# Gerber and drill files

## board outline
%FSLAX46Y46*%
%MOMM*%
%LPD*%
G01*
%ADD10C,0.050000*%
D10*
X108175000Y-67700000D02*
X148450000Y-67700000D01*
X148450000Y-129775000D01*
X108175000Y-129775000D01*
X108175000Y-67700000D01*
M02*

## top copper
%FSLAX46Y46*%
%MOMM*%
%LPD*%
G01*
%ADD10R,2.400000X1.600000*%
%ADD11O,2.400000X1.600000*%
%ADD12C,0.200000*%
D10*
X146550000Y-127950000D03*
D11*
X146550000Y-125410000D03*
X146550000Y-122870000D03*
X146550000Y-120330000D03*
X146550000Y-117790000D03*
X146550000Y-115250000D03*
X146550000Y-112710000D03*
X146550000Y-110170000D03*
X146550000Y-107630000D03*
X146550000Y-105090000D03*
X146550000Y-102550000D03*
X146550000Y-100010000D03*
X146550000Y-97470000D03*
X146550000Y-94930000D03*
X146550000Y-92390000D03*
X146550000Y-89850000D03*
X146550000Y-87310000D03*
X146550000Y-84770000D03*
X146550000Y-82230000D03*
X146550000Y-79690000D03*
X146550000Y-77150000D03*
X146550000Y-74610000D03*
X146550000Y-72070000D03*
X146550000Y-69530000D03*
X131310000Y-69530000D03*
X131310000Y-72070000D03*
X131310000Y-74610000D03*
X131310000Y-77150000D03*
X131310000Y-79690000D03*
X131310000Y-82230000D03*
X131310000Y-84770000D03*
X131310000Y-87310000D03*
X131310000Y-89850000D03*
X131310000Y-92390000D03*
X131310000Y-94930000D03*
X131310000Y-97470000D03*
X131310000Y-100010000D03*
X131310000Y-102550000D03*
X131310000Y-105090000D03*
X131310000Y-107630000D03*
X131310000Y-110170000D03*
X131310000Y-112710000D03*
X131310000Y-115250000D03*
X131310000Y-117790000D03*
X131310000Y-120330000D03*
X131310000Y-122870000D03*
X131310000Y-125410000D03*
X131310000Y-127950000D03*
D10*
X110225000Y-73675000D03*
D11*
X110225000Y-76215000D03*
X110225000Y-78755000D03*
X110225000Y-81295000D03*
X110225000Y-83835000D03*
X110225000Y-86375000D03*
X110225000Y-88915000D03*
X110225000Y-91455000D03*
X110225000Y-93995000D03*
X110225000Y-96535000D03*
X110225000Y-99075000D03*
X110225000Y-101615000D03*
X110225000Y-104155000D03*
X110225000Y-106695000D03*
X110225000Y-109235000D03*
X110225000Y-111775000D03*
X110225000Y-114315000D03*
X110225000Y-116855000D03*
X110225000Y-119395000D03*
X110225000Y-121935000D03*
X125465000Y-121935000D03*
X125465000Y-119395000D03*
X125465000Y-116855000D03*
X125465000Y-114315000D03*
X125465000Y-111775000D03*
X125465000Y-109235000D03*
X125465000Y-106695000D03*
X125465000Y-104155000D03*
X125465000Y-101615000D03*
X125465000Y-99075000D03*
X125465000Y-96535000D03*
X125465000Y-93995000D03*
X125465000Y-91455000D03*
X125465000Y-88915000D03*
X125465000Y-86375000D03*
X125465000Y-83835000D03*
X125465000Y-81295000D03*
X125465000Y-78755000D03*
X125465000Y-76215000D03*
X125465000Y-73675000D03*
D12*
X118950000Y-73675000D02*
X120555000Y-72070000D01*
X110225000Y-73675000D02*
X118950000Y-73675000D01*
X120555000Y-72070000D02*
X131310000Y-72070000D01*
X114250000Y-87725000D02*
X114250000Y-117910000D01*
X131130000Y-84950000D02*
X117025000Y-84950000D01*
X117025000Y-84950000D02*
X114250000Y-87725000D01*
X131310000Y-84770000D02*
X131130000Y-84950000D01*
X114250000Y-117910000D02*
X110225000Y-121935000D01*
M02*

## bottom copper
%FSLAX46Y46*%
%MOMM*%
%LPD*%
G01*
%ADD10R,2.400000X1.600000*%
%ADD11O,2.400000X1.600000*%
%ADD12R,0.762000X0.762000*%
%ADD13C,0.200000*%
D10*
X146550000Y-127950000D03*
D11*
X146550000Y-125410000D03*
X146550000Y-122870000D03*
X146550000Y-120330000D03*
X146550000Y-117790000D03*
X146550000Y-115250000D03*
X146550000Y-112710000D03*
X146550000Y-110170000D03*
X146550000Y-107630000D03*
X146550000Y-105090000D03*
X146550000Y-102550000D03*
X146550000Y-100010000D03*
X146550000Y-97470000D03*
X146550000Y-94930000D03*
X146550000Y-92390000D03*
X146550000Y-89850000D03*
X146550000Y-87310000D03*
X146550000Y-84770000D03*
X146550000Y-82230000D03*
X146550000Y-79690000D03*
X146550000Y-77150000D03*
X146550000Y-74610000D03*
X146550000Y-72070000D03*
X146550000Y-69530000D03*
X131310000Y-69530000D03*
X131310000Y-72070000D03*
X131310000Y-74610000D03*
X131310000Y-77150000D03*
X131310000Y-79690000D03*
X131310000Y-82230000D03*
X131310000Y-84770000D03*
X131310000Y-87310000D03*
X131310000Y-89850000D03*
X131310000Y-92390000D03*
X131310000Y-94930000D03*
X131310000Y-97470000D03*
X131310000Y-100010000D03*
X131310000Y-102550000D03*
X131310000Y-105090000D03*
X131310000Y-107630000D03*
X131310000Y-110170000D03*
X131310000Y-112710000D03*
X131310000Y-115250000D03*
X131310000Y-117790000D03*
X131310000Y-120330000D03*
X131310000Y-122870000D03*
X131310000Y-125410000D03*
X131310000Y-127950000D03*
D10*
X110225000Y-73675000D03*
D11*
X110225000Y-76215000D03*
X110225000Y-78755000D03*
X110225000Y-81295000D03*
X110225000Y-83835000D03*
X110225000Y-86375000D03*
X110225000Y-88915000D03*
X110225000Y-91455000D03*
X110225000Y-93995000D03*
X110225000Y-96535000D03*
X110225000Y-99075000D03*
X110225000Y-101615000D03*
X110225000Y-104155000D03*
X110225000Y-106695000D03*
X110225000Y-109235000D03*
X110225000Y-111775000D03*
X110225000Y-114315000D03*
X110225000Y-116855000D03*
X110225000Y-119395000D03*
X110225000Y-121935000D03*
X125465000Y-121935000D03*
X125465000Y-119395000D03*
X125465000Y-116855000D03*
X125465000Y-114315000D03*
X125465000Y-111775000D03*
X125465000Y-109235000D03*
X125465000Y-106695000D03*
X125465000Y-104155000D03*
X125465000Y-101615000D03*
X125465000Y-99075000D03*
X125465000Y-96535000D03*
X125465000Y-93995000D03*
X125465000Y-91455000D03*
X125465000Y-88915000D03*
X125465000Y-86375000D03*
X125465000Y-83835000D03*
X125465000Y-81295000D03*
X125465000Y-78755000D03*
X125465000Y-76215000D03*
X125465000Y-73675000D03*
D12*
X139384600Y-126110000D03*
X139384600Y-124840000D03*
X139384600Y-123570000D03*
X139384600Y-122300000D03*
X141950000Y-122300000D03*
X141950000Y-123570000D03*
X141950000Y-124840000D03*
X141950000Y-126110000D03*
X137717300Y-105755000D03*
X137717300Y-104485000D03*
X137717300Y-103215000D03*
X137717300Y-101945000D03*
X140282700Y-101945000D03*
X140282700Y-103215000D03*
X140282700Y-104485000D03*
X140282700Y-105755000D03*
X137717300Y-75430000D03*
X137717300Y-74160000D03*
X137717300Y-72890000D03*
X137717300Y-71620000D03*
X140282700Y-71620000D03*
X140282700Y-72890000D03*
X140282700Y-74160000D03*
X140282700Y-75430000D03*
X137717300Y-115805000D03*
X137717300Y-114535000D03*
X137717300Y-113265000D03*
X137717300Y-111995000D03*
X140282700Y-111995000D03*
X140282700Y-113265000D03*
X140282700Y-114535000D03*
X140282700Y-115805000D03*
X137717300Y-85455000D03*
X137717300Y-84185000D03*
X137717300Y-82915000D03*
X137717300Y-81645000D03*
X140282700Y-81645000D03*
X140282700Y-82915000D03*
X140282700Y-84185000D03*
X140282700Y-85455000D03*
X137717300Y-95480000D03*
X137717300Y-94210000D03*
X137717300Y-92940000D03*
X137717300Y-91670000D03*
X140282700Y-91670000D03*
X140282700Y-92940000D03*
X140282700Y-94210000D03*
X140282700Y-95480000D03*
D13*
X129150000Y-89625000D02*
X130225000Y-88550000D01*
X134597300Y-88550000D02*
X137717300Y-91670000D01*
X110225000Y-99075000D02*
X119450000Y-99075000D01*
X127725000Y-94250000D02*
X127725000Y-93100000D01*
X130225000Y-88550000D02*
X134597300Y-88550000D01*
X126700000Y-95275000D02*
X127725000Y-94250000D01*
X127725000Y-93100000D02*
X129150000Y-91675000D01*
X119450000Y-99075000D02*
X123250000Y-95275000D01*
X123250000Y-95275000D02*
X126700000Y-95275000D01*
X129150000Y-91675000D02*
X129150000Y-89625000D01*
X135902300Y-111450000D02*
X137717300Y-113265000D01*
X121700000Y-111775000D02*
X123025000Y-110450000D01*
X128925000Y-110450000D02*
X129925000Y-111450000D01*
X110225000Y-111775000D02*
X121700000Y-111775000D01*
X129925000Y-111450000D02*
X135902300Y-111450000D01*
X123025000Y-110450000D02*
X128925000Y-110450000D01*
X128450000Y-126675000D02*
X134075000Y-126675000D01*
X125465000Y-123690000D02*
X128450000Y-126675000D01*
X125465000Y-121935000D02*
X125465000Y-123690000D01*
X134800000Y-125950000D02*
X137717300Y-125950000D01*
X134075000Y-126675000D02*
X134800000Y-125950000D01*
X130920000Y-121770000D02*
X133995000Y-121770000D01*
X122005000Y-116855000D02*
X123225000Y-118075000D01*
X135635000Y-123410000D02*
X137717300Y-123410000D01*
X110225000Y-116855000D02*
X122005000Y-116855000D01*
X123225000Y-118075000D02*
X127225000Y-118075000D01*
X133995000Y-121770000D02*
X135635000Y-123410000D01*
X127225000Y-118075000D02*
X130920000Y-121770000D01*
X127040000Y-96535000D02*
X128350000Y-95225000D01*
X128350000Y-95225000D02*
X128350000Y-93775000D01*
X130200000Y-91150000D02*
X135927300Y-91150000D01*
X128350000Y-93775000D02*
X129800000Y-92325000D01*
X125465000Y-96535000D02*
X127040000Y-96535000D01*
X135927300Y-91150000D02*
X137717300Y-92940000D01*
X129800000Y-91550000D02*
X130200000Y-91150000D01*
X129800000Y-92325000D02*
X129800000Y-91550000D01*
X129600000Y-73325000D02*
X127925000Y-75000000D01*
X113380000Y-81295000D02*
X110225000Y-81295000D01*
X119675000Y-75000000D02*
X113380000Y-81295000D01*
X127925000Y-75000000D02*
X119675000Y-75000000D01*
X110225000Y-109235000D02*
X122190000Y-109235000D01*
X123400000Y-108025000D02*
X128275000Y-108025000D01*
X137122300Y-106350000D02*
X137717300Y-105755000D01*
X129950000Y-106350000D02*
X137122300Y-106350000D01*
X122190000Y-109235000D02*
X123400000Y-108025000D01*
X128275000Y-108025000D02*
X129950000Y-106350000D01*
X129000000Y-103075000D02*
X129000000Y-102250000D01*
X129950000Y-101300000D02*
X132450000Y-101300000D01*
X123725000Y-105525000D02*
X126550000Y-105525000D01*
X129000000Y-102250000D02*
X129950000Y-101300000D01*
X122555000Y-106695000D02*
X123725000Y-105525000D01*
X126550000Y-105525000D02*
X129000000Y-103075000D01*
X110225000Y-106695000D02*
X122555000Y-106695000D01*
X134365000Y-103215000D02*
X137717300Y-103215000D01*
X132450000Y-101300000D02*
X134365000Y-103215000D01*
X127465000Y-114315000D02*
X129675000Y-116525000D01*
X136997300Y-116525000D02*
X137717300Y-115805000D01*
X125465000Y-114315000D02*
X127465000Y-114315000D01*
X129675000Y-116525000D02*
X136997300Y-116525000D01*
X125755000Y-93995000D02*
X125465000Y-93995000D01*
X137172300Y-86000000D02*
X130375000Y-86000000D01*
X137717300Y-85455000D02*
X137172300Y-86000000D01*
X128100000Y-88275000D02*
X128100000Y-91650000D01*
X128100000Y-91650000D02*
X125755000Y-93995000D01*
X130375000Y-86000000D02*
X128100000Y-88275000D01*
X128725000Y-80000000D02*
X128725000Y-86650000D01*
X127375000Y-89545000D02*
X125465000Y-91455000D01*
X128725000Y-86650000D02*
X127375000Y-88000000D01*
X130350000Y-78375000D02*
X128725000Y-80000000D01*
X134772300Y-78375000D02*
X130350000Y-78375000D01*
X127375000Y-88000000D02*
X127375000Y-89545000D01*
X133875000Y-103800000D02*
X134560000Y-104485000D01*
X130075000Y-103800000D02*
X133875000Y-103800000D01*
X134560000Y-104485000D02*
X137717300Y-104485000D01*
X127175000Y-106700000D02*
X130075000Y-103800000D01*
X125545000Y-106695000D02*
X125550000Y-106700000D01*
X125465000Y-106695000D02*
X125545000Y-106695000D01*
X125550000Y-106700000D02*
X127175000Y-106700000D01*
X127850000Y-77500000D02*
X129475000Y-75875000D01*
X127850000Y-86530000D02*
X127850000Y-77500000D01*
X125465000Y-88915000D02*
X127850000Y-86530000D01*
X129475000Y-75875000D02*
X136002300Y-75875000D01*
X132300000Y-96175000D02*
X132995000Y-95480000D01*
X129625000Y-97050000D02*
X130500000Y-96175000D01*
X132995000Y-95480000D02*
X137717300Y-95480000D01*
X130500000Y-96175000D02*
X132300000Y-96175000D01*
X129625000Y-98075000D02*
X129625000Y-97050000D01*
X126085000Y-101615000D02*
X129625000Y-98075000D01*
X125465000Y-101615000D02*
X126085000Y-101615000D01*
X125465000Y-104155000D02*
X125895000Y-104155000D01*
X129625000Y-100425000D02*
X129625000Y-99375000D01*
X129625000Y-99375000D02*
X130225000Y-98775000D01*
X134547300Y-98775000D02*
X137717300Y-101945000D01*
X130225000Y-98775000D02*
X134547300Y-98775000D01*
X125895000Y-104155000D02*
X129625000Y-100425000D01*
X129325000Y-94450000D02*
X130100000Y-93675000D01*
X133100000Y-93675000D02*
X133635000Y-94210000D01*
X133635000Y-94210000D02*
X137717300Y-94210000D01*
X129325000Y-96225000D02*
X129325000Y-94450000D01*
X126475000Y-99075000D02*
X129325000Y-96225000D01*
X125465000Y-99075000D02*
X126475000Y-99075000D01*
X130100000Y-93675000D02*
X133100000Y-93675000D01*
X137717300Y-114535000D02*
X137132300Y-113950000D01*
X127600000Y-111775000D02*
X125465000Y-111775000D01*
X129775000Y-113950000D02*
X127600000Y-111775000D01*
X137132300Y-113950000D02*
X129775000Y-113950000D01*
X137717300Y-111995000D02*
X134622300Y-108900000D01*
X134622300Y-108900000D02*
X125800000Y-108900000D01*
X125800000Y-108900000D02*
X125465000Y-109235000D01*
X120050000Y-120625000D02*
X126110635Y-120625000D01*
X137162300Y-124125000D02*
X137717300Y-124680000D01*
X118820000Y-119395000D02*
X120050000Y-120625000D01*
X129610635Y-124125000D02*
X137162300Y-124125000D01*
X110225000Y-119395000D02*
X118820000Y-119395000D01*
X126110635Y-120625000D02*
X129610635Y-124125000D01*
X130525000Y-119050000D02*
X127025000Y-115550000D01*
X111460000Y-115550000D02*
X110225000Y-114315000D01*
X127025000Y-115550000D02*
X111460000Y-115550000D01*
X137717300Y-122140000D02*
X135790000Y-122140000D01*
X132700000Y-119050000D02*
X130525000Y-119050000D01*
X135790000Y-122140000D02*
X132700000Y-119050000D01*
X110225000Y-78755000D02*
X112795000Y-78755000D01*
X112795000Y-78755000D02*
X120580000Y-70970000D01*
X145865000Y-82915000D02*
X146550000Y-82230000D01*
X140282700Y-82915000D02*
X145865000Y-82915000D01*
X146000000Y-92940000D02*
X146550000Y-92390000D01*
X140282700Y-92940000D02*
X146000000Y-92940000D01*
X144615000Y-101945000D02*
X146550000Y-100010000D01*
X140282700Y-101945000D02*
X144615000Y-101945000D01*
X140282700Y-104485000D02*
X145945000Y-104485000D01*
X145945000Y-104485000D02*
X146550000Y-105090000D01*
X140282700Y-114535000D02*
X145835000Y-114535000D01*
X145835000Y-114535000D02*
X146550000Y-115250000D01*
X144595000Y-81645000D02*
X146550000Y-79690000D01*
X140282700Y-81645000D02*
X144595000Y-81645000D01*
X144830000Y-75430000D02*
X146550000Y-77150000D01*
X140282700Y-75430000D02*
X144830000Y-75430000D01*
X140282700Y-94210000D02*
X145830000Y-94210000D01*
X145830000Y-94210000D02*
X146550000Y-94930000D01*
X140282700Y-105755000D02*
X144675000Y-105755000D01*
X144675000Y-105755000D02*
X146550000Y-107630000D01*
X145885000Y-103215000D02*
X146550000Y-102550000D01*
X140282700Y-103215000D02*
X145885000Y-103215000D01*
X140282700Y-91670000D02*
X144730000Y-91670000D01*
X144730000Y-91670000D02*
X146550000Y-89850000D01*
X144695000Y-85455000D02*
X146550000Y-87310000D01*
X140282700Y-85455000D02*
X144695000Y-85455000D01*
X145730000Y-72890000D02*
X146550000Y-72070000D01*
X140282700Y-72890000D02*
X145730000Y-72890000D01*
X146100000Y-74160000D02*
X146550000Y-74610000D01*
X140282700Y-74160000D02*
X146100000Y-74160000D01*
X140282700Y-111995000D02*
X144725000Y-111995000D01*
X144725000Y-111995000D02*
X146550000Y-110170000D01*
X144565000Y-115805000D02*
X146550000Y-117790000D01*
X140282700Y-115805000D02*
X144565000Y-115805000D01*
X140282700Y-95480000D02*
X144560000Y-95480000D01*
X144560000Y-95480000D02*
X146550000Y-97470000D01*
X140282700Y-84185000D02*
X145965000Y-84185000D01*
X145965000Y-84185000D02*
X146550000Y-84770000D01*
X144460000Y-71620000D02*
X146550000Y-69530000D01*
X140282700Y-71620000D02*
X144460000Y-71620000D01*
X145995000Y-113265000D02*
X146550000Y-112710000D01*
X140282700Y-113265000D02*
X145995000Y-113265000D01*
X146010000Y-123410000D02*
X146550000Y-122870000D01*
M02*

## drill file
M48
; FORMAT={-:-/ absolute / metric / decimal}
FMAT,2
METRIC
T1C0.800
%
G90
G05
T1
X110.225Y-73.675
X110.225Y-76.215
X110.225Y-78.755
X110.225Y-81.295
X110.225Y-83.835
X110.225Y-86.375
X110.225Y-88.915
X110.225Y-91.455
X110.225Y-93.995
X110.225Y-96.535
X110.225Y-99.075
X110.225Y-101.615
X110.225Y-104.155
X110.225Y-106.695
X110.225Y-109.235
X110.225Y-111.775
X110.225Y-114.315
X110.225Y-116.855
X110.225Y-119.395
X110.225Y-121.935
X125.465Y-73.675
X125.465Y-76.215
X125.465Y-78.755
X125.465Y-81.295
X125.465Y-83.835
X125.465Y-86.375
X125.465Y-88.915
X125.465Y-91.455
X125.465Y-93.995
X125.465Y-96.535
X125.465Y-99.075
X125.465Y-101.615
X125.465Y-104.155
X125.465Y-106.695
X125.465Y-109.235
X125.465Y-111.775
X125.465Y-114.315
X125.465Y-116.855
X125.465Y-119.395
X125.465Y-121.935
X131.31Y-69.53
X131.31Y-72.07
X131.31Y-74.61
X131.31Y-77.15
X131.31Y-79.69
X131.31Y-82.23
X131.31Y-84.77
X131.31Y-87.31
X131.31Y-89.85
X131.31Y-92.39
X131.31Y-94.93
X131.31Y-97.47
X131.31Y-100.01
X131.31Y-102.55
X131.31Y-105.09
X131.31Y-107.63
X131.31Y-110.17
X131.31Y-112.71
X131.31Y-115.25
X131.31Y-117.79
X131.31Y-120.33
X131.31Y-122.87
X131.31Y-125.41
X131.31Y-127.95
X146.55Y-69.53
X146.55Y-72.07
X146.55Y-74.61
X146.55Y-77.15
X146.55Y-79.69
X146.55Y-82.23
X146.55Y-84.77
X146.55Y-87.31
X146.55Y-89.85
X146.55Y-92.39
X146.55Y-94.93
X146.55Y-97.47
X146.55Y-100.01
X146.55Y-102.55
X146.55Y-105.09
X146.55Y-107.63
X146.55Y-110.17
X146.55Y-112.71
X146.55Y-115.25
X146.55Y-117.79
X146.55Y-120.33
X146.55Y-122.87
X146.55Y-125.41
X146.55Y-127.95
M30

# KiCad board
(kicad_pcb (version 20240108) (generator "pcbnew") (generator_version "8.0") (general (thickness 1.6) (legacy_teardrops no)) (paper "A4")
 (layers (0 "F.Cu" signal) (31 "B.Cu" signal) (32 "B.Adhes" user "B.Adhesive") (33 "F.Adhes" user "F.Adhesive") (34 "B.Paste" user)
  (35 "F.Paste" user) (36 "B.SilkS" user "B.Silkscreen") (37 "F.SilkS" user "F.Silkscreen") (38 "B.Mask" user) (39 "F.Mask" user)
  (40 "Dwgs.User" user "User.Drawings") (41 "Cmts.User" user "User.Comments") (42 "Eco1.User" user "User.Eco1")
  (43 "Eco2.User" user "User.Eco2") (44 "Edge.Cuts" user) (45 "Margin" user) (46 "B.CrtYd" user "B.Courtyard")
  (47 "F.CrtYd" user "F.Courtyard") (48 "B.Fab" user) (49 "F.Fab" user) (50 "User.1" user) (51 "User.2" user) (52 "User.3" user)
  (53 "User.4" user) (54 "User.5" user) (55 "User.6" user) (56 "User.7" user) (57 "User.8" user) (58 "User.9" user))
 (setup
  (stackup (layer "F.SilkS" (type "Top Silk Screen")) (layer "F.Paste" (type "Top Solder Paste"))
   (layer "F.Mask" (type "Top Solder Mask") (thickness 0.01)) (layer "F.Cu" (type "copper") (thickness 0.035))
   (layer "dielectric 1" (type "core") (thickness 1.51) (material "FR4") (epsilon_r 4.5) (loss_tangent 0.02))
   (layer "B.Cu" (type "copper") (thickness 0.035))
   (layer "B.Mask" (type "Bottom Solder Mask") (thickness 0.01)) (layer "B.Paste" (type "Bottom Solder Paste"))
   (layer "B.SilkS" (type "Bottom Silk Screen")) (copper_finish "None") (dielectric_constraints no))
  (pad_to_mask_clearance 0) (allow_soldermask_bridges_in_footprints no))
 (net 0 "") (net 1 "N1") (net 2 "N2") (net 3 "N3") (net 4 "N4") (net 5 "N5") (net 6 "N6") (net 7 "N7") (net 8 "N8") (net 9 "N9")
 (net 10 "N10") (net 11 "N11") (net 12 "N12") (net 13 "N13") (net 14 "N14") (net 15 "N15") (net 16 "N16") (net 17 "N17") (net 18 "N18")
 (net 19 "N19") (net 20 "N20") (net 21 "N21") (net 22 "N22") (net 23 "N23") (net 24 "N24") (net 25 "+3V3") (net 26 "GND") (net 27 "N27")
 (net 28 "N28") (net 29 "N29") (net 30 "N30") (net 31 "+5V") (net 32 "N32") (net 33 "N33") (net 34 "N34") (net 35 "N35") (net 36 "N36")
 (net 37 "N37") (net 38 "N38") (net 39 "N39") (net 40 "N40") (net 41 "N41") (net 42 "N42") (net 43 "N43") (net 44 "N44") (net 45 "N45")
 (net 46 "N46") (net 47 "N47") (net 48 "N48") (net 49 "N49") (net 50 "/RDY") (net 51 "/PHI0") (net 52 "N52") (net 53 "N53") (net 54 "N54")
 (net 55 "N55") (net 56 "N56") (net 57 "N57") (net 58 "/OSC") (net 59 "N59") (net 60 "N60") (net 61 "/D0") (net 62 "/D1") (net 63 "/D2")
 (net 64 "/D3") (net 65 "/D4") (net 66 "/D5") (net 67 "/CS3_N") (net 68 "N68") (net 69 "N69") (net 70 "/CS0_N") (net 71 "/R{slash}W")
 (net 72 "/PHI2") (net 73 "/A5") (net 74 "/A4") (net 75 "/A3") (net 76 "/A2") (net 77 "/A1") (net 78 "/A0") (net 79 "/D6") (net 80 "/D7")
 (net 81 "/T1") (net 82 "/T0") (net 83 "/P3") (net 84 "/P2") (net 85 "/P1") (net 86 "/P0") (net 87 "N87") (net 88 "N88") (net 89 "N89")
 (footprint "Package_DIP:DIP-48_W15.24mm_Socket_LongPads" (layer "F.Cu") (at 146.55 127.95 180)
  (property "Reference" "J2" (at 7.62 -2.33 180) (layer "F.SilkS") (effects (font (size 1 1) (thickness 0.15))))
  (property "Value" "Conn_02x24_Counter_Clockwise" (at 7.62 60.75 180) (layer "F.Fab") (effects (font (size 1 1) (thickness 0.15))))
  (pad "1" thru_hole rect (at 0 0 180) (size 2.4 1.6) (drill 0.8) (layers "*.Cu" "*.Mask") (remove_unused_layers no) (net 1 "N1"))
  (pad "2" thru_hole oval (at 0 2.54 180) (size 2.4 1.6) (drill 0.8) (layers "*.Cu" "*.Mask") (remove_unused_layers no) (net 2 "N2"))
  (pad "3" thru_hole oval (at 0 5.08 180) (size 2.4 1.6) (drill 0.8) (layers "*.Cu" "*.Mask") (remove_unused_layers no) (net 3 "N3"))
  (pad "4" thru_hole oval (at 0 7.62 180) (size 2.4 1.6) (drill 0.8) (layers "*.Cu" "*.Mask") (remove_unused_layers no) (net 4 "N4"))
  (pad "5" thru_hole oval (at 0 10.16 180) (size 2.4 1.6) (drill 0.8) (layers "*.Cu" "*.Mask") (remove_unused_layers no) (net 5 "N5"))
  (pad "6" thru_hole oval (at 0 12.7 180) (size 2.4 1.6) (drill 0.8) (layers "*.Cu" "*.Mask") (remove_unused_layers no) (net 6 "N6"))
  (pad "7" thru_hole oval (at 0 15.24 180) (size 2.4 1.6) (drill 0.8) (layers "*.Cu" "*.Mask") (remove_unused_layers no) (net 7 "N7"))
  (pad "8" thru_hole oval (at 0 17.78 180) (size 2.4 1.6) (drill 0.8) (layers "*.Cu" "*.Mask") (remove_unused_layers no) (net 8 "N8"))
  (pad "9" thru_hole oval (at 0 20.32 180) (size 2.4 1.6) (drill 0.8) (layers "*.Cu" "*.Mask") (remove_unused_layers no) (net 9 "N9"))
  (pad "10" thru_hole oval (at 0 22.86 180) (size 2.4 1.6) (drill 0.8) (layers "*.Cu" "*.Mask") (remove_unused_layers no) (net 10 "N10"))
  (pad "11" thru_hole oval (at 0 25.4 180) (size 2.4 1.6) (drill 0.8) (layers "*.Cu" "*.Mask") (remove_unused_layers no) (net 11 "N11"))
  (pad "12" thru_hole oval (at 0 27.94 180) (size 2.4 1.6) (drill 0.8) (layers "*.Cu" "*.Mask") (remove_unused_layers no) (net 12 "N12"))
  (pad "13" thru_hole oval (at 0 30.48 180) (size 2.4 1.6) (drill 0.8) (layers "*.Cu" "*.Mask") (remove_unused_layers no) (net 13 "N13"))
  (pad "14" thru_hole oval (at 0 33.02 180) (size 2.4 1.6) (drill 0.8) (layers "*.Cu" "*.Mask") (remove_unused_layers no) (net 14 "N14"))
  (pad "15" thru_hole oval (at 0 35.56 180) (size 2.4 1.6) (drill 0.8) (layers "*.Cu" "*.Mask") (remove_unused_layers no) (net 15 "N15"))
  (pad "16" thru_hole oval (at 0 38.1 180) (size 2.4 1.6) (drill 0.8) (layers "*.Cu" "*.Mask") (remove_unused_layers no) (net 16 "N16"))
  (pad "17" thru_hole oval (at 0 40.64 180) (size 2.4 1.6) (drill 0.8) (layers "*.Cu" "*.Mask") (remove_unused_layers no) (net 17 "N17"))
  (pad "18" thru_hole oval (at 0 43.18 180) (size 2.4 1.6) (drill 0.8) (layers "*.Cu" "*.Mask") (remove_unused_layers no) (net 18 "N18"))
  (pad "19" thru_hole oval (at 0 45.72 180) (size 2.4 1.6) (drill 0.8) (layers "*.Cu" "*.Mask") (remove_unused_layers no) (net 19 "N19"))
  (pad "20" thru_hole oval (at 0 48.26 180) (size 2.4 1.6) (drill 0.8) (layers "*.Cu" "*.Mask") (remove_unused_layers no) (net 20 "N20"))
  (pad "21" thru_hole oval (at 0 50.8 180) (size 2.4 1.6) (drill 0.8) (layers "*.Cu" "*.Mask") (remove_unused_layers no) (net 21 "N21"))
  (pad "22" thru_hole oval (at 0 53.34 180) (size 2.4 1.6) (drill 0.8) (layers "*.Cu" "*.Mask") (remove_unused_layers no) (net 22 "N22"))
  (pad "23" thru_hole oval (at 0 55.88 180) (size 2.4 1.6) (drill 0.8) (layers "*.Cu" "*.Mask") (remove_unused_layers no) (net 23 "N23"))
  (pad "24" thru_hole oval (at 0 58.42 180) (size 2.4 1.6) (drill 0.8) (layers "*.Cu" "*.Mask") (remove_unused_layers no) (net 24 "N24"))
  (pad "25" thru_hole oval (at 15.24 58.42 180) (size 2.4 1.6) (drill 0.8) (layers "*.Cu" "*.Mask") (remove_unused_layers no)
   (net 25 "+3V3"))
  (pad "26" thru_hole oval (at 15.24 55.88 180) (size 2.4 1.6) (drill 0.8) (layers "*.Cu" "*.Mask") (remove_unused_layers no) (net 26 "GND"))
  (pad "27" thru_hole oval (at 15.24 53.34 180) (size 2.4 1.6) (drill 0.8) (layers "*.Cu" "*.Mask") (remove_unused_layers no) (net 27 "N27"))
  (pad "28" thru_hole oval (at 15.24 50.8 180) (size 2.4 1.6) (drill 0.8) (layers "*.Cu" "*.Mask") (remove_unused_layers no) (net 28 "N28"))
  (pad "29" thru_hole oval (at 15.24 48.26 180) (size 2.4 1.6) (drill 0.8) (layers "*.Cu" "*.Mask") (remove_unused_layers no) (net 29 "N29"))
  (pad "30" thru_hole oval (at 15.24 45.72 180) (size 2.4 1.6) (drill 0.8) (layers "*.Cu" "*.Mask") (remove_unused_layers no) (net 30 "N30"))
  (pad "31" thru_hole oval (at 15.24 43.18 180) (size 2.4 1.6) (drill 0.8) (layers "*.Cu" "*.Mask") (remove_unused_layers no) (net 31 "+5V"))
  (pad "32" thru_hole oval (at 15.24 40.64 180) (size 2.4 1.6) (drill 0.8) (layers "*.Cu" "*.Mask") (remove_unused_layers no) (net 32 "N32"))
  (pad "33" thru_hole oval (at 15.24 38.1 180) (size 2.4 1.6) (drill 0.8) (layers "*.Cu" "*.Mask") (remove_unused_layers no) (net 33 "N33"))
  (pad "34" thru_hole oval (at 15.24 35.56 180) (size 2.4 1.6) (drill 0.8) (layers "*.Cu" "*.Mask") (remove_unused_layers no) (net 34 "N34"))
  (pad "35" thru_hole oval (at 15.24 33.02 180) (size 2.4 1.6) (drill 0.8) (layers "*.Cu" "*.Mask") (remove_unused_layers no) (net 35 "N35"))
  (pad "36" thru_hole oval (at 15.24 30.48 180) (size 2.4 1.6) (drill 0.8) (layers "*.Cu" "*.Mask") (remove_unused_layers no) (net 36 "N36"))
  (pad "37" thru_hole oval (at 15.24 27.94 180) (size 2.4 1.6) (drill 0.8) (layers "*.Cu" "*.Mask") (remove_unused_layers no) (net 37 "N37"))
  (pad "38" thru_hole oval (at 15.24 25.4 180) (size 2.4 1.6) (drill 0.8) (layers "*.Cu" "*.Mask") (remove_unused_layers no) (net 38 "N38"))
  (pad "39" thru_hole oval (at 15.24 22.86 180) (size 2.4 1.6) (drill 0.8) (layers "*.Cu" "*.Mask") (remove_unused_layers no) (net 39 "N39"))
  (pad "40" thru_hole oval (at 15.24 20.32 180) (size 2.4 1.6) (drill 0.8) (layers "*.Cu" "*.Mask") (remove_unused_layers no) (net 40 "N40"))
  (pad "41" thru_hole oval (at 15.24 17.78 180) (size 2.4 1.6) (drill 0.8) (layers "*.Cu" "*.Mask") (remove_unused_layers no) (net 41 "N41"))
  (pad "42" thru_hole oval (at 15.24 15.24 180) (size 2.4 1.6) (drill 0.8) (layers "*.Cu" "*.Mask") (remove_unused_layers no) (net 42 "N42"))
  (pad "43" thru_hole oval (at 15.24 12.7 180) (size 2.4 1.6) (drill 0.8) (layers "*.Cu" "*.Mask") (remove_unused_layers no) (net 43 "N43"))
  (pad "44" thru_hole oval (at 15.24 10.16 180) (size 2.4 1.6) (drill 0.8) (layers "*.Cu" "*.Mask") (remove_unused_layers no) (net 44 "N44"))
  (pad "45" thru_hole oval (at 15.24 7.62 180) (size 2.4 1.6) (drill 0.8) (layers "*.Cu" "*.Mask") (remove_unused_layers no) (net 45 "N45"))
  (pad "46" thru_hole oval (at 15.24 5.08 180) (size 2.4 1.6) (drill 0.8) (layers "*.Cu" "*.Mask") (remove_unused_layers no) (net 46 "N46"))
  (pad "47" thru_hole oval (at 15.24 2.54 180) (size 2.4 1.6) (drill 0.8) (layers "*.Cu" "*.Mask") (remove_unused_layers no) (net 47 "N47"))
  (pad "48" thru_hole oval (at 15.24 0 180) (size 2.4 1.6) (drill 0.8) (layers "*.Cu" "*.Mask") (remove_unused_layers no) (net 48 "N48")))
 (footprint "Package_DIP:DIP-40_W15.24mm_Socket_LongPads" (layer "F.Cu") (at 110.225 73.675)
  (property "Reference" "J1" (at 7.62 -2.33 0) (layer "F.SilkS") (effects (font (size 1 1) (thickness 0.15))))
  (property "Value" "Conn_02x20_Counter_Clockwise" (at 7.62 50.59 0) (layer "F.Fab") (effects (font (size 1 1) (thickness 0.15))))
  (pad "1" thru_hole rect (at 0 0) (size 2.4 1.6) (drill 0.8) (layers "*.Cu" "*.Mask") (remove_unused_layers no) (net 26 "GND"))
  (pad "2" thru_hole oval (at 0 2.54) (size 2.4 1.6) (drill 0.8) (layers "*.Cu" "*.Mask") (remove_unused_layers no) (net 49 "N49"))
  (pad "3" thru_hole oval (at 0 5.08) (size 2.4 1.6) (drill 0.8) (layers "*.Cu" "*.Mask") (remove_unused_layers no) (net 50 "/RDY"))
  (pad "4" thru_hole oval (at 0 7.62) (size 2.4 1.6) (drill 0.8) (layers "*.Cu" "*.Mask") (remove_unused_layers no) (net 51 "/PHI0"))
  (pad "5" thru_hole oval (at 0 10.16) (size 2.4 1.6) (drill 0.8) (layers "*.Cu" "*.Mask") (remove_unused_layers no) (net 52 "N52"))
  (pad "6" thru_hole oval (at 0 12.7) (size 2.4 1.6) (drill 0.8) (layers "*.Cu" "*.Mask") (remove_unused_layers no) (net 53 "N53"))
  (pad "7" thru_hole oval (at 0 15.24) (size 2.4 1.6) (drill 0.8) (layers "*.Cu" "*.Mask") (remove_unused_layers no) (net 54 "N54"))
  (pad "8" thru_hole oval (at 0 17.78) (size 2.4 1.6) (drill 0.8) (layers "*.Cu" "*.Mask") (remove_unused_layers no) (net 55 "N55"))
  (pad "9" thru_hole oval (at 0 20.32) (size 2.4 1.6) (drill 0.8) (layers "*.Cu" "*.Mask") (remove_unused_layers no) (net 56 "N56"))
  (pad "10" thru_hole oval (at 0 22.86) (size 2.4 1.6) (drill 0.8) (layers "*.Cu" "*.Mask") (remove_unused_layers no) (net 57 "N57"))
  (pad "11" thru_hole oval (at 0 25.4) (size 2.4 1.6) (drill 0.8) (layers "*.Cu" "*.Mask") (remove_unused_layers no) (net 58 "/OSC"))
  (pad "12" thru_hole oval (at 0 27.94) (size 2.4 1.6) (drill 0.8) (layers "*.Cu" "*.Mask") (remove_unused_layers no) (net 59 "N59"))
  (pad "13" thru_hole oval (at 0 30.48) (size 2.4 1.6) (drill 0.8) (layers "*.Cu" "*.Mask") (remove_unused_layers no) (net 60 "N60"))
  (pad "14" thru_hole oval (at 0 33.02) (size 2.4 1.6) (drill 0.8) (layers "*.Cu" "*.Mask") (remove_unused_layers no) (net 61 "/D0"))
  (pad "15" thru_hole oval (at 0 35.56) (size 2.4 1.6) (drill 0.8) (layers "*.Cu" "*.Mask") (remove_unused_layers no) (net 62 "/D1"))
  (pad "16" thru_hole oval (at 0 38.1) (size 2.4 1.6) (drill 0.8) (layers "*.Cu" "*.Mask") (remove_unused_layers no) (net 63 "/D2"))
  (pad "17" thru_hole oval (at 0 40.64) (size 2.4 1.6) (drill 0.8) (layers "*.Cu" "*.Mask") (remove_unused_layers no) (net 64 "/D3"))
  (pad "18" thru_hole oval (at 0 43.18) (size 2.4 1.6) (drill 0.8) (layers "*.Cu" "*.Mask") (remove_unused_layers no) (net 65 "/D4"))
  (pad "19" thru_hole oval (at 0 45.72) (size 2.4 1.6) (drill 0.8) (layers "*.Cu" "*.Mask") (remove_unused_layers no) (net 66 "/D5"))
  (pad "20" thru_hole oval (at 0 48.26) (size 2.4 1.6) (drill 0.8) (layers "*.Cu" "*.Mask") (remove_unused_layers no) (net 31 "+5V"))
  (pad "21" thru_hole oval (at 15.24 48.26) (size 2.4 1.6) (drill 0.8) (layers "*.Cu" "*.Mask") (remove_unused_layers no) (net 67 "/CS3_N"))
  (pad "22" thru_hole oval (at 15.24 45.72) (size 2.4 1.6) (drill 0.8) (layers "*.Cu" "*.Mask") (remove_unused_layers no) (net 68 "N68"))
  (pad "23" thru_hole oval (at 15.24 43.18) (size 2.4 1.6) (drill 0.8) (layers "*.Cu" "*.Mask") (remove_unused_layers no) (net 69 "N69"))
  (pad "24" thru_hole oval (at 15.24 40.64) (size 2.4 1.6) (drill 0.8) (layers "*.Cu" "*.Mask") (remove_unused_layers no) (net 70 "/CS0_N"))
  (pad "25" thru_hole oval (at 15.24 38.1) (size 2.4 1.6) (drill 0.8) (layers "*.Cu" "*.Mask") (remove_unused_layers no)
   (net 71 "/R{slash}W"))
  (pad "26" thru_hole oval (at 15.24 35.56) (size 2.4 1.6) (drill 0.8) (layers "*.Cu" "*.Mask") (remove_unused_layers no) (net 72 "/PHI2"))
  (pad "27" thru_hole oval (at 15.24 33.02) (size 2.4 1.6) (drill 0.8) (layers "*.Cu" "*.Mask") (remove_unused_layers no) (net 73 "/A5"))
  (pad "28" thru_hole oval (at 15.24 30.48) (size 2.4 1.6) (drill 0.8) (layers "*.Cu" "*.Mask") (remove_unused_layers no) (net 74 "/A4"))
  (pad "29" thru_hole oval (at 15.24 27.94) (size 2.4 1.6) (drill 0.8) (layers "*.Cu" "*.Mask") (remove_unused_layers no) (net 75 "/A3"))
  (pad "30" thru_hole oval (at 15.24 25.4) (size 2.4 1.6) (drill 0.8) (layers "*.Cu" "*.Mask") (remove_unused_layers no) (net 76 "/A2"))
  (pad "31" thru_hole oval (at 15.24 22.86) (size 2.4 1.6) (drill 0.8) (layers "*.Cu" "*.Mask") (remove_unused_layers no) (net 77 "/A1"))
  (pad "32" thru_hole oval (at 15.24 20.32) (size 2.4 1.6) (drill 0.8) (layers "*.Cu" "*.Mask") (remove_unused_layers no) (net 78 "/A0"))
  (pad "33" thru_hole oval (at 15.24 17.78) (size 2.4 1.6) (drill 0.8) (layers "*.Cu" "*.Mask") (remove_unused_layers no) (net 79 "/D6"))
  (pad "34" thru_hole oval (at 15.24 15.24) (size 2.4 1.6) (drill 0.8) (layers "*.Cu" "*.Mask") (remove_unused_layers no) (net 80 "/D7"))
  (pad "35" thru_hole oval (at 15.24 12.7) (size 2.4 1.6) (drill 0.8) (layers "*.Cu" "*.Mask") (remove_unused_layers no) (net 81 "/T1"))
  (pad "36" thru_hole oval (at 15.24 10.16) (size 2.4 1.6) (drill 0.8) (layers "*.Cu" "*.Mask") (remove_unused_layers no) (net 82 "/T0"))
  (pad "37" thru_hole oval (at 15.24 7.62) (size 2.4 1.6) (drill 0.8) (layers "*.Cu" "*.Mask") (remove_unused_layers no) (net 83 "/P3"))
  (pad "38" thru_hole oval (at 15.24 5.08) (size 2.4 1.6) (drill 0.8) (layers "*.Cu" "*.Mask") (remove_unused_layers no) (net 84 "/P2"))
  (pad "39" thru_hole oval (at 15.24 2.54) (size 2.4 1.6) (drill 0.8) (layers "*.Cu" "*.Mask") (remove_unused_layers no) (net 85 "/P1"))
  (pad "40" thru_hole oval (at 15.24 0) (size 2.4 1.6) (drill 0.8) (layers "*.Cu" "*.Mask") (remove_unused_layers no) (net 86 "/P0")))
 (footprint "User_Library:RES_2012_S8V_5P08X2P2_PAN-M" (layer "B.Cu") (at 140.6673 124.205)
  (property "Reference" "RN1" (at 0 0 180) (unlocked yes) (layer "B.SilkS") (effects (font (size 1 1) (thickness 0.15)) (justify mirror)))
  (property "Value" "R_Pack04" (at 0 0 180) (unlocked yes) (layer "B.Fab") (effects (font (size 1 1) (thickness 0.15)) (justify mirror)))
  (pad "1" smd rect (at -1.2827 1.905) (size 0.762 0.762) (layers "B.Cu" "B.Paste" "B.Mask") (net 30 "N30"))
  (pad "2" smd rect (at -1.2827 0.635) (size 0.762 0.762) (layers "B.Cu" "B.Paste" "B.Mask") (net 29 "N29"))
  (pad "3" smd rect (at -1.2827 -0.635) (size 0.762 0.762) (layers "B.Cu" "B.Paste" "B.Mask") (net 28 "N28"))
  (pad "4" smd rect (at -1.2827 -1.905) (size 0.762 0.762) (layers "B.Cu" "B.Paste" "B.Mask") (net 27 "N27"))
  (pad "5" smd rect (at 1.2827 -1.905) (size 0.762 0.762) (layers "B.Cu" "B.Paste" "B.Mask") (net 64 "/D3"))
  (pad "6" smd rect (at 1.2827 -0.635) (size 0.762 0.762) (layers "B.Cu" "B.Paste" "B.Mask") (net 65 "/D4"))
  (pad "7" smd rect (at 1.2827 0.635) (size 0.762 0.762) (layers "B.Cu" "B.Paste" "B.Mask") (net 66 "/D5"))
  (pad "8" smd rect (at 1.2827 1.905) (size 0.762 0.762) (layers "B.Cu" "B.Paste" "B.Mask") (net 67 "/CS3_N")))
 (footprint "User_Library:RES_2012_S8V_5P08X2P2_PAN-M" (layer "B.Cu") (at 139 103.85)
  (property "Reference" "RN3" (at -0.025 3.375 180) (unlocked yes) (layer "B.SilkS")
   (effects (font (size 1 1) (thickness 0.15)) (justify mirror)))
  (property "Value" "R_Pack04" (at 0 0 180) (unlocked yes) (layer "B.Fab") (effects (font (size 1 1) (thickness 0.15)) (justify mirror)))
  (pad "1" smd rect (at -1.2827 1.905) (size 0.762 0.762) (layers "B.Cu" "B.Paste" "B.Mask") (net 62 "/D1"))
  (pad "2" smd rect (at -1.2827 0.635) (size 0.762 0.762) (layers "B.Cu" "B.Paste" "B.Mask") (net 73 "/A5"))
  (pad "3" smd rect (at -1.2827 -0.635) (size 0.762 0.762) (layers "B.Cu" "B.Paste" "B.Mask") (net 61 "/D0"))
  (pad "4" smd rect (at -1.2827 -1.905) (size 0.762 0.762) (layers "B.Cu" "B.Paste" "B.Mask") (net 74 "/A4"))
  (pad "5" smd rect (at 1.2827 -1.905) (size 0.762 0.762) (layers "B.Cu" "B.Paste" "B.Mask") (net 12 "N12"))
  (pad "6" smd rect (at 1.2827 -0.635) (size 0.762 0.762) (layers "B.Cu" "B.Paste" "B.Mask") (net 11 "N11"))
  (pad "7" smd rect (at 1.2827 0.635) (size 0.762 0.762) (layers "B.Cu" "B.Paste" "B.Mask") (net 10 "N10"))
  (pad "8" smd rect (at 1.2827 1.905) (size 0.762 0.762) (layers "B.Cu" "B.Paste" "B.Mask") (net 9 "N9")))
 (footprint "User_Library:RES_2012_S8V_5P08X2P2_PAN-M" (layer "B.Cu") (at 139 73.525)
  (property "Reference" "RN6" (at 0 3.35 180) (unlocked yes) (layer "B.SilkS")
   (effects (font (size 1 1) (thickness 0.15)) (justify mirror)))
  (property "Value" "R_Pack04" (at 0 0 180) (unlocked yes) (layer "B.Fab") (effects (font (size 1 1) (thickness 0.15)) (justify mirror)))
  (pad "1" smd rect (at -1.2827 1.905) (size 0.762 0.762) (layers "B.Cu" "B.Paste" "B.Mask") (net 50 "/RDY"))
  (pad "2" smd rect (at -1.2827 0.635) (size 0.762 0.762) (layers "B.Cu" "B.Paste" "B.Mask") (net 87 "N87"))
  (pad "3" smd rect (at -1.2827 -0.635) (size 0.762 0.762) (layers "B.Cu" "B.Paste" "B.Mask") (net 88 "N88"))
  (pad "4" smd rect (at -1.2827 -1.905) (size 0.762 0.762) (layers "B.Cu" "B.Paste" "B.Mask") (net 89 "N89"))
  (pad "5" smd rect (at 1.2827 -1.905) (size 0.762 0.762) (layers "B.Cu" "B.Paste" "B.Mask") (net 24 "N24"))
  (pad "6" smd rect (at 1.2827 -0.635) (size 0.762 0.762) (layers "B.Cu" "B.Paste" "B.Mask") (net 23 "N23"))
  (pad "7" smd rect (at 1.2827 0.635) (size 0.762 0.762) (layers "B.Cu" "B.Paste" "B.Mask") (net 22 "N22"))
  (pad "8" smd rect (at 1.2827 1.905) (size 0.762 0.762) (layers "B.Cu" "B.Paste" "B.Mask") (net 21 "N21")))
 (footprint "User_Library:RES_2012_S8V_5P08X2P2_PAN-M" (layer "B.Cu") (at 139 113.9)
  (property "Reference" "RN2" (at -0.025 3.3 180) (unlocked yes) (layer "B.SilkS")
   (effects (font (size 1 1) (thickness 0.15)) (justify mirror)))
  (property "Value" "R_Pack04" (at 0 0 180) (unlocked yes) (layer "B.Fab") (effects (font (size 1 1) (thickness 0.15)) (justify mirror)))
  (pad "1" smd rect (at -1.2827 1.905) (size 0.762 0.762) (layers "B.Cu" "B.Paste" "B.Mask") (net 70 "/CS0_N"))
  (pad "2" smd rect (at -1.2827 0.635) (size 0.762 0.762) (layers "B.Cu" "B.Paste" "B.Mask") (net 71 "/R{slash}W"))
  (pad "3" smd rect (at -1.2827 -0.635) (size 0.762 0.762) (layers "B.Cu" "B.Paste" "B.Mask") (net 63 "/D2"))
  (pad "4" smd rect (at -1.2827 -1.905) (size 0.762 0.762) (layers "B.Cu" "B.Paste" "B.Mask") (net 72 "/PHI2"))
  (pad "5" smd rect (at 1.2827 -1.905) (size 0.762 0.762) (layers "B.Cu" "B.Paste" "B.Mask") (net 8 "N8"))
  (pad "6" smd rect (at 1.2827 -0.635) (size 0.762 0.762) (layers "B.Cu" "B.Paste" "B.Mask") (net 7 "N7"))
  (pad "7" smd rect (at 1.2827 0.635) (size 0.762 0.762) (layers "B.Cu" "B.Paste" "B.Mask") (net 6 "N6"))
  (pad "8" smd rect (at 1.2827 1.905) (size 0.762 0.762) (layers "B.Cu" "B.Paste" "B.Mask") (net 5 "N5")))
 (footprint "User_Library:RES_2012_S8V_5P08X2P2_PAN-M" (layer "B.Cu") (at 139 83.55)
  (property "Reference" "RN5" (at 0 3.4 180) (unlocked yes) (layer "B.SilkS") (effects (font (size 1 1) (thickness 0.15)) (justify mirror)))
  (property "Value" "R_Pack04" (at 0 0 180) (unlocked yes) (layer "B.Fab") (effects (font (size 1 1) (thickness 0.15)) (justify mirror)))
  (pad "1" smd rect (at -1.2827 1.905) (size 0.762 0.762) (layers "B.Cu" "B.Paste" "B.Mask") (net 78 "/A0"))
  (pad "2" smd rect (at -1.2827 0.635) (size 0.762 0.762) (layers "B.Cu" "B.Paste" "B.Mask") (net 79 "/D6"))
  (pad "3" smd rect (at -1.2827 -0.635) (size 0.762 0.762) (layers "B.Cu" "B.Paste" "B.Mask") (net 80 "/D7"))
  (pad "4" smd rect (at -1.2827 -1.905) (size 0.762 0.762) (layers "B.Cu" "B.Paste" "B.Mask") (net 51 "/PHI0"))
  (pad "5" smd rect (at 1.2827 -1.905) (size 0.762 0.762) (layers "B.Cu" "B.Paste" "B.Mask") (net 20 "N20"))
  (pad "6" smd rect (at 1.2827 -0.635) (size 0.762 0.762) (layers "B.Cu" "B.Paste" "B.Mask") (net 19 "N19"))
  (pad "7" smd rect (at 1.2827 0.635) (size 0.762 0.762) (layers "B.Cu" "B.Paste" "B.Mask") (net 18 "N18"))
  (pad "8" smd rect (at 1.2827 1.905) (size 0.762 0.762) (layers "B.Cu" "B.Paste" "B.Mask") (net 17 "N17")))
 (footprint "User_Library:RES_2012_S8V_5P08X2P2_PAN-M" (layer "B.Cu") (at 139 93.575)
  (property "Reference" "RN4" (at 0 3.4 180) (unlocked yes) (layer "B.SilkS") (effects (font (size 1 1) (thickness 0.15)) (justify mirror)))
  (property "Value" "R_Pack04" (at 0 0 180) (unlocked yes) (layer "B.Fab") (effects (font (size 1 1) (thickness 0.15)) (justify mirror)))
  (pad "1" smd rect (at -1.2827 1.905) (size 0.762 0.762) (layers "B.Cu" "B.Paste" "B.Mask") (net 75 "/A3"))
  (pad "2" smd rect (at -1.2827 0.635) (size 0.762 0.762) (layers "B.Cu" "B.Paste" "B.Mask") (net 76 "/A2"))
  (pad "3" smd rect (at -1.2827 -0.635) (size 0.762 0.762) (layers "B.Cu" "B.Paste" "B.Mask") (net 77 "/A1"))
  (pad "4" smd rect (at -1.2827 -1.905) (size 0.762 0.762) (layers "B.Cu" "B.Paste" "B.Mask") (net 58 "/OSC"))
  (pad "5" smd rect (at 1.2827 -1.905) (size 0.762 0.762) (layers "B.Cu" "B.Paste" "B.Mask") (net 16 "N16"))
  (pad "6" smd rect (at 1.2827 -0.635) (size 0.762 0.762) (layers "B.Cu" "B.Paste" "B.Mask") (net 15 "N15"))
  (pad "7" smd rect (at 1.2827 0.635) (size 0.762 0.762) (layers "B.Cu" "B.Paste" "B.Mask") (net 14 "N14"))
  (pad "8" smd rect (at 1.2827 1.905) (size 0.762 0.762) (layers "B.Cu" "B.Paste" "B.Mask") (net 13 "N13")))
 (gr_rect (start 108.175 67.7) (end 148.45 129.775) (stroke (width 0.05) (type default)) (fill none) (layer "Edge.Cuts"))
 (segment (start 129.15 89.625) (end 130.225 88.55) (width 0.2) (layer "B.Cu") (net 58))
 (segment (start 134.5973 88.55) (end 137.7173 91.67) (width 0.2) (layer "B.Cu") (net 58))
 (segment (start 110.225 99.075) (end 119.45 99.075) (width 0.2) (layer "B.Cu") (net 58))
 (segment (start 127.725 94.25) (end 127.725 93.1) (width 0.2) (layer "B.Cu") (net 58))
 (segment (start 130.225 88.55) (end 134.5973 88.55) (width 0.2) (layer "B.Cu") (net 58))
 (segment (start 126.7 95.275) (end 127.725 94.25) (width 0.2) (layer "B.Cu") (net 58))
 (segment (start 127.725 93.1) (end 129.15 91.675) (width 0.2) (layer "B.Cu") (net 58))
 (segment (start 119.45 99.075) (end 123.25 95.275) (width 0.2) (layer "B.Cu") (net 58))
 (segment (start 123.25 95.275) (end 126.7 95.275) (width 0.2) (layer "B.Cu") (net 58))
 (segment (start 129.15 91.675) (end 129.15 89.625) (width 0.2) (layer "B.Cu") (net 58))
 (segment (start 135.9023 111.45) (end 137.7173 113.265) (width 0.2) (layer "B.Cu") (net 63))
 (segment (start 121.7 111.775) (end 123.025 110.45) (width 0.2) (layer "B.Cu") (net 63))
 (segment (start 128.925 110.45) (end 129.925 111.45) (width 0.2) (layer "B.Cu") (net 63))
 (segment (start 110.225 111.775) (end 121.7 111.775) (width 0.2) (layer "B.Cu") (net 63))
 (segment (start 129.925 111.45) (end 135.9023 111.45) (width 0.2) (layer "B.Cu") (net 63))
 (segment (start 123.025 110.45) (end 128.925 110.45) (width 0.2) (layer "B.Cu") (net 63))
 (segment (start 128.45 126.675) (end 134.075 126.675) (width 0.2) (layer "B.Cu") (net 67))
 (segment (start 125.465 123.69) (end 128.45 126.675) (width 0.2) (layer "B.Cu") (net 67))
 (segment (start 125.465 121.935) (end 125.465 123.69) (width 0.2) (layer "B.Cu") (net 67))
 (segment (start 134.8 125.95) (end 137.7173 125.95) (width 0.2) (layer "B.Cu") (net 67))
 (segment (start 134.075 126.675) (end 134.8 125.95) (width 0.2) (layer "B.Cu") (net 67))
 (segment (start 130.92 121.77) (end 133.995 121.77) (width 0.2) (layer "B.Cu") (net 65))
 (segment (start 122.005 116.855) (end 123.225 118.075) (width 0.2) (layer "B.Cu") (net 65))
 (segment (start 135.635 123.41) (end 137.7173 123.41) (width 0.2) (layer "B.Cu") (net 65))
 (segment (start 110.225 116.855) (end 122.005 116.855) (width 0.2) (layer "B.Cu") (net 65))
 (segment (start 123.225 118.075) (end 127.225 118.075) (width 0.2) (layer "B.Cu") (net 65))
 (segment (start 133.995 121.77) (end 135.635 123.41) (width 0.2) (layer "B.Cu") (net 65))
 (segment (start 127.225 118.075) (end 130.92 121.77) (width 0.2) (layer "B.Cu") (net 65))
 (segment (start 127.04 96.535) (end 128.35 95.225) (width 0.2) (layer "B.Cu") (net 77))
 (segment (start 128.35 95.225) (end 128.35 93.775) (width 0.2) (layer "B.Cu") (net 77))
 (segment (start 130.2 91.15) (end 135.9273 91.15) (width 0.2) (layer "B.Cu") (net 77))
 (segment (start 128.35 93.775) (end 129.8 92.325) (width 0.2) (layer "B.Cu") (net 77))
 (segment (start 125.465 96.535) (end 127.04 96.535) (width 0.2) (layer "B.Cu") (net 77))
 (segment (start 135.9273 91.15) (end 137.7173 92.94) (width 0.2) (layer "B.Cu") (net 77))
 (segment (start 129.8 91.55) (end 130.2 91.15) (width 0.2) (layer "B.Cu") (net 77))
 (segment (start 129.8 92.325) (end 129.8 91.55) (width 0.2) (layer "B.Cu") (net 77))
 (segment (start 129.6 73.325) (end 127.925 75) (width 0.2) (layer "B.Cu") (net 51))
 (segment (start 113.38 81.295) (end 110.225 81.295) (width 0.2) (layer "B.Cu") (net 51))
 (segment (start 119.675 75) (end 113.38 81.295) (width 0.2) (layer "B.Cu") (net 51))
 (segment (start 127.925 75) (end 119.675 75) (width 0.2) (layer "B.Cu") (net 51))
 (segment (start 110.225 109.235) (end 122.19 109.235) (width 0.2) (layer "B.Cu") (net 62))
 (segment (start 123.4 108.025) (end 128.275 108.025) (width 0.2) (layer "B.Cu") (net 62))
 (segment (start 137.1223 106.35) (end 137.7173 105.755) (width 0.2) (layer "B.Cu") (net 62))
 (segment (start 129.95 106.35) (end 137.1223 106.35) (width 0.2) (layer "B.Cu") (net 62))
 (segment (start 122.19 109.235) (end 123.4 108.025) (width 0.2) (layer "B.Cu") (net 62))
 (segment (start 128.275 108.025) (end 129.95 106.35) (width 0.2) (layer "B.Cu") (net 62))
 (segment (start 129 103.075) (end 129 102.25) (width 0.2) (layer "B.Cu") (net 61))
 (segment (start 129.95 101.3) (end 132.45 101.3) (width 0.2) (layer "B.Cu") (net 61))
 (segment (start 123.725 105.525) (end 126.55 105.525) (width 0.2) (layer "B.Cu") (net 61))
 (segment (start 129 102.25) (end 129.95 101.3) (width 0.2) (layer "B.Cu") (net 61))
 (segment (start 122.555 106.695) (end 123.725 105.525) (width 0.2) (layer "B.Cu") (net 61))
 (segment (start 126.55 105.525) (end 129 103.075) (width 0.2) (layer "B.Cu") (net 61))
 (segment (start 110.225 106.695) (end 122.555 106.695) (width 0.2) (layer "B.Cu") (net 61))
 (segment (start 134.365 103.215) (end 137.7173 103.215) (width 0.2) (layer "B.Cu") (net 61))
 (segment (start 132.45 101.3) (end 134.365 103.215) (width 0.2) (layer "B.Cu") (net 61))
 (segment (start 127.465 114.315) (end 129.675 116.525) (width 0.2) (layer "B.Cu") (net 70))
 (segment (start 136.9973 116.525) (end 137.7173 115.805) (width 0.2) (layer "B.Cu") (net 70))
 (segment (start 125.465 114.315) (end 127.465 114.315) (width 0.2) (layer "B.Cu") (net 70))
 (segment (start 129.675 116.525) (end 136.9973 116.525) (width 0.2) (layer "B.Cu") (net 70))
 (segment (start 125.755 93.995) (end 125.465 93.995) (width 0.2) (layer "B.Cu") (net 78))
 (segment (start 137.1723 86) (end 130.375 86) (width 0.2) (layer "B.Cu") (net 78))
 (segment (start 137.7173 85.455) (end 137.1723 86) (width 0.2) (layer "B.Cu") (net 78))
 (segment (start 128.1 88.275) (end 128.1 91.65) (width 0.2) (layer "B.Cu") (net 78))
 (segment (start 128.1 91.65) (end 125.755 93.995) (width 0.2) (layer "B.Cu") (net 78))
 (segment (start 130.375 86) (end 128.1 88.275) (width 0.2) (layer "B.Cu") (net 78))
 (segment (start 128.725 80) (end 128.725 86.65) (width 0.2) (layer "B.Cu") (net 79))
 (segment (start 127.375 89.545) (end 125.465 91.455) (width 0.2) (layer "B.Cu") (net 79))
 (segment (start 128.725 86.65) (end 127.375 88) (width 0.2) (layer "B.Cu") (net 79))
 (segment (start 130.35 78.375) (end 128.725 80) (width 0.2) (layer "B.Cu") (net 79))
 (segment (start 134.7723 78.375) (end 130.35 78.375) (width 0.2) (layer "B.Cu") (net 79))
 (segment (start 127.375 88) (end 127.375 89.545) (width 0.2) (layer "B.Cu") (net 79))
 (segment (start 133.875 103.8) (end 134.56 104.485) (width 0.2) (layer "B.Cu") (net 73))
 (segment (start 130.075 103.8) (end 133.875 103.8) (width 0.2) (layer "B.Cu") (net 73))
 (segment (start 134.56 104.485) (end 137.7173 104.485) (width 0.2) (layer "B.Cu") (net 73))
 (segment (start 127.175 106.7) (end 130.075 103.8) (width 0.2) (layer "B.Cu") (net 73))
 (segment (start 125.545 106.695) (end 125.55 106.7) (width 0.2) (layer "B.Cu") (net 73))
 (segment (start 125.465 106.695) (end 125.545 106.695) (width 0.2) (layer "B.Cu") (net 73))
 (segment (start 125.55 106.7) (end 127.175 106.7) (width 0.2) (layer "B.Cu") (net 73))
 (segment (start 127.85 77.5) (end 129.475 75.875) (width 0.2) (layer "B.Cu") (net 80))
 (segment (start 127.85 86.53) (end 127.85 77.5) (width 0.2) (layer "B.Cu") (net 80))
 (segment (start 125.465 88.915) (end 127.85 86.53) (width 0.2) (layer "B.Cu") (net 80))
 (segment (start 129.475 75.875) (end 136.0023 75.875) (width 0.2) (layer "B.Cu") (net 80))
 (segment (start 132.3 96.175) (end 132.995 95.48) (width 0.2) (layer "B.Cu") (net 75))
 (segment (start 129.625 97.05) (end 130.5 96.175) (width 0.2) (layer "B.Cu") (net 75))
 (segment (start 132.995 95.48) (end 137.7173 95.48) (width 0.2) (layer "B.Cu") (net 75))
 (segment (start 130.5 96.175) (end 132.3 96.175) (width 0.2) (layer "B.Cu") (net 75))
 (segment (start 129.625 98.075) (end 129.625 97.05) (width 0.2) (layer "B.Cu") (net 75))
 (segment (start 126.085 101.615) (end 129.625 98.075) (width 0.2) (layer "B.Cu") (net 75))
 (segment (start 125.465 101.615) (end 126.085 101.615) (width 0.2) (layer "B.Cu") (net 75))
 (segment (start 125.465 104.155) (end 125.895 104.155) (width 0.2) (layer "B.Cu") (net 74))
 (segment (start 129.625 100.425) (end 129.625 99.375) (width 0.2) (layer "B.Cu") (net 74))
 (segment (start 129.625 99.375) (end 130.225 98.775) (width 0.2) (layer "B.Cu") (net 74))
 (segment (start 134.5473 98.775) (end 137.7173 101.945) (width 0.2) (layer "B.Cu") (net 74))
 (segment (start 130.225 98.775) (end 134.5473 98.775) (width 0.2) (layer "B.Cu") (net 74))
 (segment (start 125.895 104.155) (end 129.625 100.425) (width 0.2) (layer "B.Cu") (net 74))
 (segment (start 129.325 94.45) (end 130.1 93.675) (width 0.2) (layer "B.Cu") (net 76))
 (segment (start 133.1 93.675) (end 133.635 94.21) (width 0.2) (layer "B.Cu") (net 76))
 (segment (start 133.635 94.21) (end 137.7173 94.21) (width 0.2) (layer "B.Cu") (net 76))
 (segment (start 129.325 96.225) (end 129.325 94.45) (width 0.2) (layer "B.Cu") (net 76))
 (segment (start 126.475 99.075) (end 129.325 96.225) (width 0.2) (layer "B.Cu") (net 76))
 (segment (start 125.465 99.075) (end 126.475 99.075) (width 0.2) (layer "B.Cu") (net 76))
 (segment (start 130.1 93.675) (end 133.1 93.675) (width 0.2) (layer "B.Cu") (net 76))
 (segment (start 118.95 73.675) (end 120.555 72.07) (width 0.2) (layer "F.Cu") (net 26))
 (segment (start 110.225 73.675) (end 118.95 73.675) (width 0.2) (layer "F.Cu") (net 26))
 (segment (start 120.555 72.07) (end 131.31 72.07) (width 0.2) (layer "F.Cu") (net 26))
 (segment (start 137.7173 114.535) (end 137.1323 113.95) (width 0.2) (layer "B.Cu") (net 71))
 (segment (start 127.6 111.775) (end 125.465 111.775) (width 0.2) (layer "B.Cu") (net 71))
 (segment (start 129.775 113.95) (end 127.6 111.775) (width 0.2) (layer "B.Cu") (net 71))
 (segment (start 137.1323 113.95) (end 129.775 113.95) (width 0.2) (layer "B.Cu") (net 71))
 (segment (start 137.7173 111.995) (end 134.6223 108.9) (width 0.2) (layer "B.Cu") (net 72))
 (segment (start 134.6223 108.9) (end 125.8 108.9) (width 0.2) (layer "B.Cu") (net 72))
 (segment (start 125.8 108.9) (end 125.465 109.235) (width 0.2) (layer "B.Cu") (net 72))
 (segment (start 120.05 120.625) (end 126.110635 120.625) (width 0.2) (layer "B.Cu") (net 66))
 (segment (start 137.1623 124.125) (end 137.7173 124.68) (width 0.2) (layer "B.Cu") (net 66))
 (segment (start 118.82 119.395) (end 120.05 120.625) (width 0.2) (layer "B.Cu") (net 66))
 (segment (start 129.610635 124.125) (end 137.1623 124.125) (width 0.2) (layer "B.Cu") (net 66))
 (segment (start 110.225 119.395) (end 118.82 119.395) (width 0.2) (layer "B.Cu") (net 66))
 (segment (start 126.110635 120.625) (end 129.610635 124.125) (width 0.2) (layer "B.Cu") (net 66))
 (segment (start 130.525 119.05) (end 127.025 115.55) (width 0.2) (layer "B.Cu") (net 64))
 (segment (start 111.46 115.55) (end 110.225 114.315) (width 0.2) (layer "B.Cu") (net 64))
 (segment (start 127.025 115.55) (end 111.46 115.55) (width 0.2) (layer "B.Cu") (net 64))
 (segment (start 137.7173 122.14) (end 135.79 122.14) (width 0.2) (layer "B.Cu") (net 64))
 (segment (start 132.7 119.05) (end 130.525 119.05) (width 0.2) (layer "B.Cu") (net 64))
 (segment (start 135.79 122.14) (end 132.7 119.05) (width 0.2) (layer "B.Cu") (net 64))
 (segment (start 114.25 87.725) (end 114.25 117.91) (width 0.2) (layer "F.Cu") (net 31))
 (segment (start 131.13 84.95) (end 117.025 84.95) (width 0.2) (layer "F.Cu") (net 31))
 (segment (start 117.025 84.95) (end 114.25 87.725) (width 0.2) (layer "F.Cu") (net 31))
 (segment (start 131.31 84.77) (end 131.13 84.95) (width 0.2) (layer "F.Cu") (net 31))
 (segment (start 114.25 117.91) (end 110.225 121.935) (width 0.2) (layer "F.Cu") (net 31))
 (segment (start 110.225 78.755) (end 112.795 78.755) (width 0.2) (layer "B.Cu") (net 50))
 (segment (start 112.795 78.755) (end 120.58 70.97) (width 0.2) (layer "B.Cu") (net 50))
 (segment (start 145.865 82.915) (end 146.55 82.23) (width 0.2) (layer "B.Cu") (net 19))
 (segment (start 140.2827 82.915) (end 145.865 82.915) (width 0.2) (layer "B.Cu") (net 19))
 (segment (start 146 92.94) (end 146.55 92.39) (width 0.2) (layer "B.Cu") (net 15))
 (segment (start 140.2827 92.94) (end 146 92.94) (width 0.2) (layer "B.Cu") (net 15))
 (segment (start 144.615 101.945) (end 146.55 100.01) (width 0.2) (layer "B.Cu") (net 12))
 (segment (start 140.2827 101.945) (end 144.615 101.945) (width 0.2) (layer "B.Cu") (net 12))
 (segment (start 140.2827 104.485) (end 145.945 104.485) (width 0.2) (layer "B.Cu") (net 10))
 (segment (start 145.945 104.485) (end 146.55 105.09) (width 0.2) (layer "B.Cu") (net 10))
 (segment (start 140.2827 114.535) (end 145.835 114.535) (width 0.2) (layer "B.Cu") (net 6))
 (segment (start 145.835 114.535) (end 146.55 115.25) (width 0.2) (layer "B.Cu") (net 6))
 (segment (start 144.595 81.645) (end 146.55 79.69) (width 0.2) (layer "B.Cu") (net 20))
 (segment (start 140.2827 81.645) (end 144.595 81.645) (width 0.2) (layer "B.Cu") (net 20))
 (segment (start 144.83 75.43) (end 146.55 77.15) (width 0.2) (layer "B.Cu") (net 21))
 (segment (start 140.2827 75.43) (end 144.83 75.43) (width 0.2) (layer "B.Cu") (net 21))
 (segment (start 140.2827 94.21) (end 145.83 94.21) (width 0.2) (layer "B.Cu") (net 14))
 (segment (start 145.83 94.21) (end 146.55 94.93) (width 0.2) (layer "B.Cu") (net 14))
 (segment (start 140.2827 105.755) (end 144.675 105.755) (width 0.2) (layer "B.Cu") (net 9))
 (segment (start 144.675 105.755) (end 146.55 107.63) (width 0.2) (layer "B.Cu") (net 9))
 (segment (start 145.885 103.215) (end 146.55 102.55) (width 0.2) (layer "B.Cu") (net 11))
 (segment (start 140.2827 103.215) (end 145.885 103.215) (width 0.2) (layer "B.Cu") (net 11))
 (segment (start 140.2827 91.67) (end 144.73 91.67) (width 0.2) (layer "B.Cu") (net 16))
 (segment (start 144.73 91.67) (end 146.55 89.85) (width 0.2) (layer "B.Cu") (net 16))
 (segment (start 144.695 85.455) (end 146.55 87.31) (width 0.2) (layer "B.Cu") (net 17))
 (segment (start 140.2827 85.455) (end 144.695 85.455) (width 0.2) (layer "B.Cu") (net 17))
 (segment (start 145.73 72.89) (end 146.55 72.07) (width 0.2) (layer "B.Cu") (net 23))
 (segment (start 140.2827 72.89) (end 145.73 72.89) (width 0.2) (layer "B.Cu") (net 23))
 (segment (start 146.1 74.16) (end 146.55 74.61) (width 0.2) (layer "B.Cu") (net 22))
 (segment (start 140.2827 74.16) (end 146.1 74.16) (width 0.2) (layer "B.Cu") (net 22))
 (segment (start 140.2827 111.995) (end 144.725 111.995) (width 0.2) (layer "B.Cu") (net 8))
 (segment (start 144.725 111.995) (end 146.55 110.17) (width 0.2) (layer "B.Cu") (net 8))
 (segment (start 144.565 115.805) (end 146.55 117.79) (width 0.2) (layer "B.Cu") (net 5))
 (segment (start 140.2827 115.805) (end 144.565 115.805) (width 0.2) (layer "B.Cu") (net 5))
 (segment (start 140.2827 95.48) (end 144.56 95.48) (width 0.2) (layer "B.Cu") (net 13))
 (segment (start 144.56 95.48) (end 146.55 97.47) (width 0.2) (layer "B.Cu") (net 13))
 (segment (start 140.2827 84.185) (end 145.965 84.185) (width 0.2) (layer "B.Cu") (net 18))
 (segment (start 145.965 84.185) (end 146.55 84.77) (width 0.2) (layer "B.Cu") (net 18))
 (segment (start 144.46 71.62) (end 146.55 69.53) (width 0.2) (layer "B.Cu") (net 24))
 (segment (start 140.2827 71.62) (end 144.46 71.62) (width 0.2) (layer "B.Cu") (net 24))
 (segment (start 145.995 113.265) (end 146.55 112.71) (width 0.2) (layer "B.Cu") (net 7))
 (segment (start 140.2827 113.265) (end 145.995 113.265) (width 0.2) (layer "B.Cu") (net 7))
 (segment (start 146.01 123.41) (end 146.55 122.87) (width 0.2) (layer "B.Cu") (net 3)))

